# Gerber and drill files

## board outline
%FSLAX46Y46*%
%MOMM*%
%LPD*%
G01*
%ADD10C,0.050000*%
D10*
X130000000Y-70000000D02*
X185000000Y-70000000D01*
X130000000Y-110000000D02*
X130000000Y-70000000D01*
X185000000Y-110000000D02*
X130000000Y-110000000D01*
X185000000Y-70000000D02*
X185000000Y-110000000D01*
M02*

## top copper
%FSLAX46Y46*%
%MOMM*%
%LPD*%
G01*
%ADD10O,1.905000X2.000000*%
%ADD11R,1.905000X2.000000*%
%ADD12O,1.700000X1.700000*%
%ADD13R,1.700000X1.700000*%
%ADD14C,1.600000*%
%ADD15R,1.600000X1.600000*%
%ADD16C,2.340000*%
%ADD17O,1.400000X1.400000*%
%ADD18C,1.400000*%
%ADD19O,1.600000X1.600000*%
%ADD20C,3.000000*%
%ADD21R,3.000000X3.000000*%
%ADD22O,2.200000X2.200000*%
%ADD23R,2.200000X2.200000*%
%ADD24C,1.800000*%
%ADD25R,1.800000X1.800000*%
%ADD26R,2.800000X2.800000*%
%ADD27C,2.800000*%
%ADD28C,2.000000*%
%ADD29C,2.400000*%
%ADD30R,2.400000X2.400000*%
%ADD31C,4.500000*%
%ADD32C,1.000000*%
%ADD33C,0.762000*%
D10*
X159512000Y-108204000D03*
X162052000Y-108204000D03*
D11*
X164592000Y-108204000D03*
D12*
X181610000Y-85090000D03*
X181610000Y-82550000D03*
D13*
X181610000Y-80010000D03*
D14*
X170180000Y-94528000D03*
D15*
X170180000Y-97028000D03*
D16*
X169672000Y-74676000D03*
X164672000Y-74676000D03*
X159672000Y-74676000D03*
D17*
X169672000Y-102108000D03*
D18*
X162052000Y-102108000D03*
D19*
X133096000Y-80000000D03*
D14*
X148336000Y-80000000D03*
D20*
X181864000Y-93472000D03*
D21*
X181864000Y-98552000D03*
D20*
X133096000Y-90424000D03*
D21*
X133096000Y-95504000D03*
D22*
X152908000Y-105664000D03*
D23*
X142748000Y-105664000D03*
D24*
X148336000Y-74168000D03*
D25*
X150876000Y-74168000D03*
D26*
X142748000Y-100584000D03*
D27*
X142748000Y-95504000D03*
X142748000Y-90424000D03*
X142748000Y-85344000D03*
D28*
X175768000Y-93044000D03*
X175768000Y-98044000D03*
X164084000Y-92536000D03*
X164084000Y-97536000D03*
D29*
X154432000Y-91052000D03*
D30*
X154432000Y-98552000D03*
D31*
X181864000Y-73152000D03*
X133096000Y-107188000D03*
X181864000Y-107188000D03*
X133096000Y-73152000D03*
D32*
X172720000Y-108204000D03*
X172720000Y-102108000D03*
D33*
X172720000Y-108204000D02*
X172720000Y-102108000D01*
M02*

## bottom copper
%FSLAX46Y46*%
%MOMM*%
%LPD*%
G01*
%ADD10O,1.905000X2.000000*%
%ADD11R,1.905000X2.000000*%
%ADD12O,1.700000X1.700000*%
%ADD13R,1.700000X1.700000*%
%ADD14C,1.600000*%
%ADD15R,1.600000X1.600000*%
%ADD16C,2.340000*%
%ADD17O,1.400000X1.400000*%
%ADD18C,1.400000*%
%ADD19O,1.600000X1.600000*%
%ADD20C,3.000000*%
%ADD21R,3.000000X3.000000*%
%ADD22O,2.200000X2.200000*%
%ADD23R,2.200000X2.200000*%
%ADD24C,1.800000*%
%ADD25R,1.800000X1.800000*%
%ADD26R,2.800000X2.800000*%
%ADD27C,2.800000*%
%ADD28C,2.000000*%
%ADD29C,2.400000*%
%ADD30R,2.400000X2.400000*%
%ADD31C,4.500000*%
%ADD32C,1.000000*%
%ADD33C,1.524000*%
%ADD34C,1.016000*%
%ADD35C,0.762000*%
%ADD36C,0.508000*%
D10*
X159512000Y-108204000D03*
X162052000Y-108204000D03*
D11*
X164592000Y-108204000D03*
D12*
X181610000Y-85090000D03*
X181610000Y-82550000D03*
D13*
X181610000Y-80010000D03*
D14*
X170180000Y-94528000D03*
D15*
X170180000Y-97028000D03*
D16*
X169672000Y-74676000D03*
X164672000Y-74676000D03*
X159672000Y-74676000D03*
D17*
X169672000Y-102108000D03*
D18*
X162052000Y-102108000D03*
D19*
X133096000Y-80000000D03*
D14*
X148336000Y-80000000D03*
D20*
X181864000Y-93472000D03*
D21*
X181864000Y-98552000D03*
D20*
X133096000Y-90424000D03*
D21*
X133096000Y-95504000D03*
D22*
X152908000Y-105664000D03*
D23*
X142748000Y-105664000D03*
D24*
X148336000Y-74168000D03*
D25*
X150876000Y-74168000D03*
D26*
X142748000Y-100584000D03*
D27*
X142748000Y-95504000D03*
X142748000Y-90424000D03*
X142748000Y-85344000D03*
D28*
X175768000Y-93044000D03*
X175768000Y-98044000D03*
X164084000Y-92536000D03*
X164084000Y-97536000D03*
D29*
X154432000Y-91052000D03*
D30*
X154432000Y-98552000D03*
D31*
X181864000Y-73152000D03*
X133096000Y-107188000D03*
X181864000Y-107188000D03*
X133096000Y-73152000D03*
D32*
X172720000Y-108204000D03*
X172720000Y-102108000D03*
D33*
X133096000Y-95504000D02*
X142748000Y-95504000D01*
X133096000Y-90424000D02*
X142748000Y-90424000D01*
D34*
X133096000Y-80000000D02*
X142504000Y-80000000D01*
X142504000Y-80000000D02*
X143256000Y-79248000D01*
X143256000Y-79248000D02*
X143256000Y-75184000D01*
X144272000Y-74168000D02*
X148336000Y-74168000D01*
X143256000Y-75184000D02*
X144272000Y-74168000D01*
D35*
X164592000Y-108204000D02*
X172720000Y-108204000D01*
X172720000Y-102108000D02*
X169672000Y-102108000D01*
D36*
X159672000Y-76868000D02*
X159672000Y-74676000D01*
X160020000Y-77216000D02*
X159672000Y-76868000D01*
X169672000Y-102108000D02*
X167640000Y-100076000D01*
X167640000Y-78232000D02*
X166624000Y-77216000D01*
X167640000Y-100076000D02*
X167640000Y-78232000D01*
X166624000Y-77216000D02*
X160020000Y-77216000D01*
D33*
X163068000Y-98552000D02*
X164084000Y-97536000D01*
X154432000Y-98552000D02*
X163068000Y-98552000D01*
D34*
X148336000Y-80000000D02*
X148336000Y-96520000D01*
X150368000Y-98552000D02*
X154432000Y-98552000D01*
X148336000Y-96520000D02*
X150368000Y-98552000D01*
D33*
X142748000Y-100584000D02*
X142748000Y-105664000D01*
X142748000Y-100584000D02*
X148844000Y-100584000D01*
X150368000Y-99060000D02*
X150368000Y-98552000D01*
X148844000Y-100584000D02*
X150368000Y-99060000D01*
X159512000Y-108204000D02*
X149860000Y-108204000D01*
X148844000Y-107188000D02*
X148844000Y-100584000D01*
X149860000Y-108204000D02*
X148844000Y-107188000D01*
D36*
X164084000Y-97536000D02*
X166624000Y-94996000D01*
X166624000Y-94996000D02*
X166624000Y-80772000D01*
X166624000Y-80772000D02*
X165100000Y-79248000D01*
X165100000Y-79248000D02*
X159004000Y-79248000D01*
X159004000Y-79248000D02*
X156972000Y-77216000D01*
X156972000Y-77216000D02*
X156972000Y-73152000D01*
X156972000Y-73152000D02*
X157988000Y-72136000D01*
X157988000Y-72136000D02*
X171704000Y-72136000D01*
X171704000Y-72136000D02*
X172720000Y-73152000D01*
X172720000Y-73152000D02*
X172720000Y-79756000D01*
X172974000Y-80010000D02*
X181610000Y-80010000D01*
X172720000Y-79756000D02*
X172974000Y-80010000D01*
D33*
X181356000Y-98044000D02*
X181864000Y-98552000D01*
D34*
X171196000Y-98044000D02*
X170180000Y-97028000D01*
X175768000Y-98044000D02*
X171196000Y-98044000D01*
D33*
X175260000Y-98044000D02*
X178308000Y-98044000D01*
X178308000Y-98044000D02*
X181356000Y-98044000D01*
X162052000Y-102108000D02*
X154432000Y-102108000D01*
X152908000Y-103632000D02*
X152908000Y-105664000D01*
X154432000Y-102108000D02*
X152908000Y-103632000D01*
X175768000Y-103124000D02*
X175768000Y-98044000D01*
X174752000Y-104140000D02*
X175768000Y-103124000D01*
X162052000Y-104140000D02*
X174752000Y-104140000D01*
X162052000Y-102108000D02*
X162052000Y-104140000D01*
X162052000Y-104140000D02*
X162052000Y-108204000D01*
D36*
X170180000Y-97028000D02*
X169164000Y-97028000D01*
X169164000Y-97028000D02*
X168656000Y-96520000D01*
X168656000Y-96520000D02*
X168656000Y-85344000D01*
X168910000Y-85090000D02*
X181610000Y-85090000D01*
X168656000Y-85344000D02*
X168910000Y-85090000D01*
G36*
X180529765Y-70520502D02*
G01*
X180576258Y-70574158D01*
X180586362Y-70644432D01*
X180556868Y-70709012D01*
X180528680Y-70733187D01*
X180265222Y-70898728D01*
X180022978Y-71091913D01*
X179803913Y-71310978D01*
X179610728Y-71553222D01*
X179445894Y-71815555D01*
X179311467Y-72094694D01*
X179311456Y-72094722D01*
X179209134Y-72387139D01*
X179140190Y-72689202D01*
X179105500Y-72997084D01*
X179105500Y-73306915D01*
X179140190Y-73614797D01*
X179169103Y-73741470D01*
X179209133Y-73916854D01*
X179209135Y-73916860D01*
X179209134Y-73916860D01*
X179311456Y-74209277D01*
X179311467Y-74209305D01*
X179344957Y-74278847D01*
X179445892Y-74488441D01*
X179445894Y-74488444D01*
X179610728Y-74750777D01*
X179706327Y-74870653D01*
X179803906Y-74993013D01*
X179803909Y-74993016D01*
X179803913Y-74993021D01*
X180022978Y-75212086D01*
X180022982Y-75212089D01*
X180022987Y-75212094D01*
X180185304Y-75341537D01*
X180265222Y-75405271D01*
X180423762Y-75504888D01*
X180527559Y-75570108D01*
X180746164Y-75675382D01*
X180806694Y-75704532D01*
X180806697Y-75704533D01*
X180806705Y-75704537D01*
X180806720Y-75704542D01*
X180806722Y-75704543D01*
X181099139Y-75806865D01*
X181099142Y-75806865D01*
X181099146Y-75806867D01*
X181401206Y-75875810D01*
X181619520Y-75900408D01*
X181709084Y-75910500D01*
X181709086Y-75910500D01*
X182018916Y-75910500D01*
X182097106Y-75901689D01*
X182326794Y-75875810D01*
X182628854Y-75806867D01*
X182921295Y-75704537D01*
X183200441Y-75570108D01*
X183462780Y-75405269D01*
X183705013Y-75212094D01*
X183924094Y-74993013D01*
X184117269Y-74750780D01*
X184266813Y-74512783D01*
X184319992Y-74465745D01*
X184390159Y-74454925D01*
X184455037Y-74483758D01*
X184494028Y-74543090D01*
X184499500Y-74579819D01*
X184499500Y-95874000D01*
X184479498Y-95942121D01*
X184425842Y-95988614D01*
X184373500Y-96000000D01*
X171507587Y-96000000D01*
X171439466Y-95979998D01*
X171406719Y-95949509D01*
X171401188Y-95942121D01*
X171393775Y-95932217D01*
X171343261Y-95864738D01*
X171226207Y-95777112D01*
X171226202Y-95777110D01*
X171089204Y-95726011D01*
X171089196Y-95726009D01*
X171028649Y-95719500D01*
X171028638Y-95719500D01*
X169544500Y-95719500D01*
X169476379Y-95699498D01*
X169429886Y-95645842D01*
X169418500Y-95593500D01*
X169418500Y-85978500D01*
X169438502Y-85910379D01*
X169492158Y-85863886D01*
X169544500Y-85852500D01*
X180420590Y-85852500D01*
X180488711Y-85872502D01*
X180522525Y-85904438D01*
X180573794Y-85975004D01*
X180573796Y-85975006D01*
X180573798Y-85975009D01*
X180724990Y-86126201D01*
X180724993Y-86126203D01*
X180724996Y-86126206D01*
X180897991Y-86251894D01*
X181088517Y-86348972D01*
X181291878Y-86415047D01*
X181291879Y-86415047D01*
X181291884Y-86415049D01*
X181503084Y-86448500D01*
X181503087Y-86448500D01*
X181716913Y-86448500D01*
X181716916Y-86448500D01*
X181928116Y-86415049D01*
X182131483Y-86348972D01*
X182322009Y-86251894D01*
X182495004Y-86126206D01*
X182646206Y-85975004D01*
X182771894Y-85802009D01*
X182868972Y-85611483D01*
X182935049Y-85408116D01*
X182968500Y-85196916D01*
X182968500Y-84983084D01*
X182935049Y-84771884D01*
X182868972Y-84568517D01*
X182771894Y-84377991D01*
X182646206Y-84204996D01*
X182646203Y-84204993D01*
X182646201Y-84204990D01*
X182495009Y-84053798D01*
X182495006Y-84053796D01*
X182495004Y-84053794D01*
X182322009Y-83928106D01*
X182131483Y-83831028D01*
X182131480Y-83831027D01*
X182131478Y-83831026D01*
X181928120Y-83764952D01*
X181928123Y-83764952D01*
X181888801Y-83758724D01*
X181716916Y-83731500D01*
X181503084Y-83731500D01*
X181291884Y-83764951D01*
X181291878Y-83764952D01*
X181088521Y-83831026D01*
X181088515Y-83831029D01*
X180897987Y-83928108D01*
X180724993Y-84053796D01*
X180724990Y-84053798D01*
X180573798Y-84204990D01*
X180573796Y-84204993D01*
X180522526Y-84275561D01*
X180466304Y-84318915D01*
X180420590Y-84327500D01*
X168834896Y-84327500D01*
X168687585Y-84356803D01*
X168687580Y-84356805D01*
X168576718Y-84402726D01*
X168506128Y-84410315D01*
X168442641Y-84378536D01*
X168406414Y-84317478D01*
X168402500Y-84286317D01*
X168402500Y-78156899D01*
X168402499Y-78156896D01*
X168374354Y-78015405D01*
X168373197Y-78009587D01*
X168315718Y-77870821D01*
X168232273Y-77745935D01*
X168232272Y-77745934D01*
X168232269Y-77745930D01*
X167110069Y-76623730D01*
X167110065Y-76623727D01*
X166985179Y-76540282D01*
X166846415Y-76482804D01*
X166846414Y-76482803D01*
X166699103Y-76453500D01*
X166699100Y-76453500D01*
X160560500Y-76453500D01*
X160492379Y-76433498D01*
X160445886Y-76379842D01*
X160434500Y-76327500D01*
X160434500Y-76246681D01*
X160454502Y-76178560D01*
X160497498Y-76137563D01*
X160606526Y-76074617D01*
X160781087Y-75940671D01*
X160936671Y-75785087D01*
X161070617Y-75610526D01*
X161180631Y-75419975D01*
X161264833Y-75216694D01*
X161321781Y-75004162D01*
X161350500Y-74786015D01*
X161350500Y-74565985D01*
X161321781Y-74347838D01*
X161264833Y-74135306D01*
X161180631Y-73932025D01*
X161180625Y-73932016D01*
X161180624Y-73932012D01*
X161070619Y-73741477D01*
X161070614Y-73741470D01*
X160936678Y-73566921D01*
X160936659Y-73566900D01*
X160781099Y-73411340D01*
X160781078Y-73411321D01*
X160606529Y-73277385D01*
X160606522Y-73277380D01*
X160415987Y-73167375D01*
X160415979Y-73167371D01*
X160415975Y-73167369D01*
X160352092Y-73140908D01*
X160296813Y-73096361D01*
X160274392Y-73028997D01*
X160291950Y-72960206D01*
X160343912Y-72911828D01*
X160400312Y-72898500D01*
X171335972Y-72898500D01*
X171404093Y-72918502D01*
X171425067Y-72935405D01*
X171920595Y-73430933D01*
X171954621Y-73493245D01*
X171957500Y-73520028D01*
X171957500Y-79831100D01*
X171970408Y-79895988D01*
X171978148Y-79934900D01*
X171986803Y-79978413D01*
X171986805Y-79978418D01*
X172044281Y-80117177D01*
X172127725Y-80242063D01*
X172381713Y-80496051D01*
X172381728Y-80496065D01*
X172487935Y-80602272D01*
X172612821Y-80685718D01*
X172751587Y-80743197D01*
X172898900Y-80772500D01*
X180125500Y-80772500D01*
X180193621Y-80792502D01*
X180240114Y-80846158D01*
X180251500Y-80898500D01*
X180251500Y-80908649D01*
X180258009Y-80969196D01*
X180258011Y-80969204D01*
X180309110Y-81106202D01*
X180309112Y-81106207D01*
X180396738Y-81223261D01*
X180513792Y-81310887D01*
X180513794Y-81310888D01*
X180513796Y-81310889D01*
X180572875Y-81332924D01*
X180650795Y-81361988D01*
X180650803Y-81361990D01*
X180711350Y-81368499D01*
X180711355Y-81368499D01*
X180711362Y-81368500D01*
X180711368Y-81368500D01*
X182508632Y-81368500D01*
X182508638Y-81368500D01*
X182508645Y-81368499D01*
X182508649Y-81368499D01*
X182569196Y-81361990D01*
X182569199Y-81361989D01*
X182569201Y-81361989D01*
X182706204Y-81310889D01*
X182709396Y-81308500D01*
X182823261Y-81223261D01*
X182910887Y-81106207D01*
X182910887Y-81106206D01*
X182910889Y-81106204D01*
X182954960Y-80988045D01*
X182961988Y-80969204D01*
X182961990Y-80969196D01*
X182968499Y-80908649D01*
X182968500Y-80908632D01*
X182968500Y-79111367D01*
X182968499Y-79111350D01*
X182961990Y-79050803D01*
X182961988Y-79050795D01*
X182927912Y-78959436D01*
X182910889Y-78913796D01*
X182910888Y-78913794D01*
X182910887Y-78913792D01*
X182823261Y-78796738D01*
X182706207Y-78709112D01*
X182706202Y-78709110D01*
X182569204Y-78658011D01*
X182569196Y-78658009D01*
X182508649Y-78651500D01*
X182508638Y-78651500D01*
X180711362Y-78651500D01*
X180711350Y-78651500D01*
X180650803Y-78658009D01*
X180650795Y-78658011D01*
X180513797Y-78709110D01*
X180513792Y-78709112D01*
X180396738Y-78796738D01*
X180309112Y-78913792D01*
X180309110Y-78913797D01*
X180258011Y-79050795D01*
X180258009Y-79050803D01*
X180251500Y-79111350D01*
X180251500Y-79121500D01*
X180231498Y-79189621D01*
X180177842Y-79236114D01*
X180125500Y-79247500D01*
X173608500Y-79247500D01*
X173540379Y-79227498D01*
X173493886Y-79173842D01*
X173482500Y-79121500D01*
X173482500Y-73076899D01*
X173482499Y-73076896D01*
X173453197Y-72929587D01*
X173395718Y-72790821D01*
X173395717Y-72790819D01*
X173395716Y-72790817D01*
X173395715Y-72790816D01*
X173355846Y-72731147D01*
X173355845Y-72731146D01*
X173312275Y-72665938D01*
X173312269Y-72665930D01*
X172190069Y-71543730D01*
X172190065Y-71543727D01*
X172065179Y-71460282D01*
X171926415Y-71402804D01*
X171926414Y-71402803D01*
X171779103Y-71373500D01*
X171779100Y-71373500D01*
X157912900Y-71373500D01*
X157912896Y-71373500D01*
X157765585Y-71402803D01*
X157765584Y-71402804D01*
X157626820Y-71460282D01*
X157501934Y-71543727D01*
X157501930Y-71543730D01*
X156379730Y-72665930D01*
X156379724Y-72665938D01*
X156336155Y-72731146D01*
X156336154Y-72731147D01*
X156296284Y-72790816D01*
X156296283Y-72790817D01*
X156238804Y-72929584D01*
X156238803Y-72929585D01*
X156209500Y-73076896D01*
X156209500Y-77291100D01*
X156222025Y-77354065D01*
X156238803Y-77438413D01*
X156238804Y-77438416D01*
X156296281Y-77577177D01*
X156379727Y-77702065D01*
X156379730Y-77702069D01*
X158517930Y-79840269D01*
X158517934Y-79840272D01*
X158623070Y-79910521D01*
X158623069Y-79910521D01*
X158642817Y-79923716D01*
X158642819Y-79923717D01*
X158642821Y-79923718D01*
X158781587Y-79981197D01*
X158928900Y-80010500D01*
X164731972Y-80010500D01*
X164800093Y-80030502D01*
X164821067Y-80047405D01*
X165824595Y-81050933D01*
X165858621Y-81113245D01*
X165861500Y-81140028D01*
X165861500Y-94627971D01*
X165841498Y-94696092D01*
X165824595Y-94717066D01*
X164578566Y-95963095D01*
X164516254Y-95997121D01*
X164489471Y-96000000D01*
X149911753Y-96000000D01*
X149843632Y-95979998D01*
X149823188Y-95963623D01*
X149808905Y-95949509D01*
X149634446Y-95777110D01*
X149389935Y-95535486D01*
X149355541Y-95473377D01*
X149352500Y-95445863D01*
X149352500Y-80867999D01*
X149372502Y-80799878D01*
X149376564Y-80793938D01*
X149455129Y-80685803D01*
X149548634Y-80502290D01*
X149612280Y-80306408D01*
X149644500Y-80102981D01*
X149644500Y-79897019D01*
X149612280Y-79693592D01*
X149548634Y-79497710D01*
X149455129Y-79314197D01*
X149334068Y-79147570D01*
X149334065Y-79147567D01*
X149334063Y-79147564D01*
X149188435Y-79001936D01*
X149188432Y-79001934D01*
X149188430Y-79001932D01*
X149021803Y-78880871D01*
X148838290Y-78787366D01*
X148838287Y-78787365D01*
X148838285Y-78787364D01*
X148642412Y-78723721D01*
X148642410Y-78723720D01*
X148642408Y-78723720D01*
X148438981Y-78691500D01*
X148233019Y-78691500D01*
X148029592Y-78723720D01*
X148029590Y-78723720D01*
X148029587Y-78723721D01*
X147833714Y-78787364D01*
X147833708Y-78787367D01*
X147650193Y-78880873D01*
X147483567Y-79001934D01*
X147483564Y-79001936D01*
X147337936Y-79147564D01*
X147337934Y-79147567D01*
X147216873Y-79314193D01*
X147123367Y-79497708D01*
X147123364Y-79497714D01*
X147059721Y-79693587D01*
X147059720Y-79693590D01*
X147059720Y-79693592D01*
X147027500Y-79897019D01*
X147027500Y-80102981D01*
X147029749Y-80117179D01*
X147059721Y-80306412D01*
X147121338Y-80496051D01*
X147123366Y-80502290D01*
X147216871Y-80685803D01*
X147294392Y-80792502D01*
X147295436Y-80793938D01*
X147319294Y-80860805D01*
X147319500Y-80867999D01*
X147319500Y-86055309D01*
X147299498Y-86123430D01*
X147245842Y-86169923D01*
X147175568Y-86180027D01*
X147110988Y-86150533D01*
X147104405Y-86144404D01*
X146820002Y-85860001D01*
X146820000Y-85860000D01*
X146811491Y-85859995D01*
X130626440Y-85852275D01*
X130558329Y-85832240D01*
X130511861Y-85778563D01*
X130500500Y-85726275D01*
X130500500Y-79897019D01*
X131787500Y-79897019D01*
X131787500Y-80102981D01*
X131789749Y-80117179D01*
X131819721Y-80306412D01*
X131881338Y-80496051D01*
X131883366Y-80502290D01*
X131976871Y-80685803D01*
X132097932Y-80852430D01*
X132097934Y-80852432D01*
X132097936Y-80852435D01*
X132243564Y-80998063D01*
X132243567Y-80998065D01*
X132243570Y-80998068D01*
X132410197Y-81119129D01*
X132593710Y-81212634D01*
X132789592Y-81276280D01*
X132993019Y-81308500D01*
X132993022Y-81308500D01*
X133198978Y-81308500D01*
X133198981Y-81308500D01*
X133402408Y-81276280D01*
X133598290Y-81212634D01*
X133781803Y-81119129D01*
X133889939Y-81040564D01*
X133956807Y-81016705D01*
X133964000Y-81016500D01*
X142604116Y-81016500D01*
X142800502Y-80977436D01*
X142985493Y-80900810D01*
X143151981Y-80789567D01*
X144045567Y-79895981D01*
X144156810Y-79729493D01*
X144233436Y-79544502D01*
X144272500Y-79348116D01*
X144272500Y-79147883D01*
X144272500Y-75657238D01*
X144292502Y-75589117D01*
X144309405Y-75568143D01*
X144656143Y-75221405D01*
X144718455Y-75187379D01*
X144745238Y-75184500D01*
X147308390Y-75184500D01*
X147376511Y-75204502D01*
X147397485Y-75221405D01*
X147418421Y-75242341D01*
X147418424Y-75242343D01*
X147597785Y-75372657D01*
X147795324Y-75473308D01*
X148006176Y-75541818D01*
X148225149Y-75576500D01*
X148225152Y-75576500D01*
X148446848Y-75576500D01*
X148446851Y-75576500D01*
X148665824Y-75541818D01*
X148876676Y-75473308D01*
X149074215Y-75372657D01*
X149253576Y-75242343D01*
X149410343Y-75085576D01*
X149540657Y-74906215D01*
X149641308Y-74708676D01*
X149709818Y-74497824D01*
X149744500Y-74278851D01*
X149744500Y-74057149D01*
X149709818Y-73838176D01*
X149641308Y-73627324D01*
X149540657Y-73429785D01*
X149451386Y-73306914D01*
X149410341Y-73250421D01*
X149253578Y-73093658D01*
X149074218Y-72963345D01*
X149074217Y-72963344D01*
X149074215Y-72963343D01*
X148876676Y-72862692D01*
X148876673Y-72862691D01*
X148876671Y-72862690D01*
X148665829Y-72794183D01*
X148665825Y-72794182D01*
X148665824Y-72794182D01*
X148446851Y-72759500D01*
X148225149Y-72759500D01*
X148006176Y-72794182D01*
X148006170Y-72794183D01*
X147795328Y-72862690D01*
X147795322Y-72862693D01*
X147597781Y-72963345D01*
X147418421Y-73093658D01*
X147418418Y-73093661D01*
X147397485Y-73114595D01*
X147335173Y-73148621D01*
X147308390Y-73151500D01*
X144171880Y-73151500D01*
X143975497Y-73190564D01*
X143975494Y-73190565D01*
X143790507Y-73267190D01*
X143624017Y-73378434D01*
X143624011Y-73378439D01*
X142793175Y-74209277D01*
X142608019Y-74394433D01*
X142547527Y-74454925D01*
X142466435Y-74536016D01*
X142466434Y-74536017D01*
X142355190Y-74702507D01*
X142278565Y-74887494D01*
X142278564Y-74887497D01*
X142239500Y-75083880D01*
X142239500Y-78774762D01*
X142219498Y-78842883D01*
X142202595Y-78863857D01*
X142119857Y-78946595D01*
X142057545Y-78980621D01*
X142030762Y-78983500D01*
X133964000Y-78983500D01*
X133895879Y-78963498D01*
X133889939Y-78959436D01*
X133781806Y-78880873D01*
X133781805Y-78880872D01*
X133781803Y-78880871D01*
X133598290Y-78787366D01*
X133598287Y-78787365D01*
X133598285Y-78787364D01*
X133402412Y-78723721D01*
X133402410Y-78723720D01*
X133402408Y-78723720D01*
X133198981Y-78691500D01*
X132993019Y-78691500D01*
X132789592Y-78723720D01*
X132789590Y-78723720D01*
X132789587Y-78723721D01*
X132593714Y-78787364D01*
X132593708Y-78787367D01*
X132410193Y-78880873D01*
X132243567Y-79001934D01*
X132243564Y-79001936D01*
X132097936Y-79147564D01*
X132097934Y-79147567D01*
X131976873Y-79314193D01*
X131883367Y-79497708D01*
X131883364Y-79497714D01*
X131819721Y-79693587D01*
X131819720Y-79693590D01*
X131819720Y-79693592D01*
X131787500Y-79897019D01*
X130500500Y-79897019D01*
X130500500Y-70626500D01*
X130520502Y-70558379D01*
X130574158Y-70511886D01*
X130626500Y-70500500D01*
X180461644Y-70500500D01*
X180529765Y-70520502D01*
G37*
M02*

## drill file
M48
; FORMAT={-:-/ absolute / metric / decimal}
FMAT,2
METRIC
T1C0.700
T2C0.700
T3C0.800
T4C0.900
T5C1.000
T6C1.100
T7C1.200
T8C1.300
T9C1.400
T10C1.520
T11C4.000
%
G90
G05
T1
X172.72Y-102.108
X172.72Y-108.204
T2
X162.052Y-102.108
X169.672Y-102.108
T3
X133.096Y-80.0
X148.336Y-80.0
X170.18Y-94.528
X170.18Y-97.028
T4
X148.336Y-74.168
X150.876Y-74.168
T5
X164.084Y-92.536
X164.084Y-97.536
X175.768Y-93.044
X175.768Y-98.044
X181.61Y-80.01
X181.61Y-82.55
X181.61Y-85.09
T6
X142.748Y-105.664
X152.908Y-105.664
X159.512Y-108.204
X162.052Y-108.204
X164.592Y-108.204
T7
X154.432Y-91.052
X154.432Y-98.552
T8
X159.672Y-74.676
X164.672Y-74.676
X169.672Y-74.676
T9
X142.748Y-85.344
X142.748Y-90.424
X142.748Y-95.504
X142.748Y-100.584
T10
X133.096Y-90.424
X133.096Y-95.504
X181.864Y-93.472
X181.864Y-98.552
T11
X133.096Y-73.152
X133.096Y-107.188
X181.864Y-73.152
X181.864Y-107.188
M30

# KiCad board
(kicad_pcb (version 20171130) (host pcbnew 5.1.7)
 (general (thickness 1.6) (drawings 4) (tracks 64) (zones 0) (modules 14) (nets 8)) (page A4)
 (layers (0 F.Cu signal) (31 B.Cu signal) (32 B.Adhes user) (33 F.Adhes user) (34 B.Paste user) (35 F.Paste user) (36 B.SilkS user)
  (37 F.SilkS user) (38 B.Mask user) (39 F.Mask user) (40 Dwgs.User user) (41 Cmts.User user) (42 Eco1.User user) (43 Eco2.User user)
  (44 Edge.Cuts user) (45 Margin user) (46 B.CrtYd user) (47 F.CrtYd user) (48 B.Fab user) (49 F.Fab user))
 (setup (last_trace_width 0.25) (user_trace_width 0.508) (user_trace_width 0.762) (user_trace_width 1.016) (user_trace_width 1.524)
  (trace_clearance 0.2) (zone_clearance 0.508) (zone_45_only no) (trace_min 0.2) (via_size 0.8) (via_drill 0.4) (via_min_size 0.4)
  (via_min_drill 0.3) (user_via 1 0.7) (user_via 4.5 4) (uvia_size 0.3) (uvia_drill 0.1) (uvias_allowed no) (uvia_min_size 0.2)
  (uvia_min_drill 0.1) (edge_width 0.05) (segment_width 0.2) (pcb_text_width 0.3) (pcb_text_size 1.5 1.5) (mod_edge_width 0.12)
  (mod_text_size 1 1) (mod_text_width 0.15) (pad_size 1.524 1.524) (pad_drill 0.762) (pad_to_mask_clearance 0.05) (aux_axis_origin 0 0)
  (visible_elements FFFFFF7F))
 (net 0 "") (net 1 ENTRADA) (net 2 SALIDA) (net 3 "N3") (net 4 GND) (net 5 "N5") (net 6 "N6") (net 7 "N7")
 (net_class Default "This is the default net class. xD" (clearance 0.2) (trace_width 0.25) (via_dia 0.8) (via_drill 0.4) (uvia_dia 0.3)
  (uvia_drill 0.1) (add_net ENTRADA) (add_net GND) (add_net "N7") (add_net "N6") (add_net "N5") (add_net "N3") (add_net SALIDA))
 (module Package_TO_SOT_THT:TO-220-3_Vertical (layer F.Cu) (at 164.592 108.204 180)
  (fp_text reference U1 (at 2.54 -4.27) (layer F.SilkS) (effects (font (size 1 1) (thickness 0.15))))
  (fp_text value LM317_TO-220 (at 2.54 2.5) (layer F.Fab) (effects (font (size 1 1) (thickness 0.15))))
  (pad 3 thru_hole oval (at 5.08 0 180) (size 1.905 2) (drill 1.1) (layers *.Cu *.Mask) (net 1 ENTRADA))
  (pad 2 thru_hole oval (at 2.54 0 180) (size 1.905 2) (drill 1.1) (layers *.Cu *.Mask) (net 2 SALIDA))
  (pad 1 thru_hole rect (at 0 0 180) (size 1.905 2) (drill 1.1) (layers *.Cu *.Mask) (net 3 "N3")))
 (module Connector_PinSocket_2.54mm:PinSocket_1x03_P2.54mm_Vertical (layer F.Cu) (at 181.61 80.01)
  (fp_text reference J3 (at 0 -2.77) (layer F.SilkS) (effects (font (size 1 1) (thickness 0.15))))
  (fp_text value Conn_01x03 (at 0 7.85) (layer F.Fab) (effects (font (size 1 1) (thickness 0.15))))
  (pad 3 thru_hole oval (at 0 5.08) (size 1.7 1.7) (drill 1) (layers *.Cu *.Mask) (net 2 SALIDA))
  (pad 2 thru_hole oval (at 0 2.54) (size 1.7 1.7) (drill 1) (layers *.Cu *.Mask) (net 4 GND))
  (pad 1 thru_hole rect (at 0 0) (size 1.7 1.7) (drill 1) (layers *.Cu *.Mask) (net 1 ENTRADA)))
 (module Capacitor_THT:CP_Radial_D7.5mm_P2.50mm (layer F.Cu) (at 170.18 97.028 90)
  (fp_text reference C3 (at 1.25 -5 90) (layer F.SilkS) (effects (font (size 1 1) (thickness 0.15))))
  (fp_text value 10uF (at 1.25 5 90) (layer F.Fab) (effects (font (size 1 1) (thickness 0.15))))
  (pad 2 thru_hole circle (at 2.5 0 90) (size 1.6 1.6) (drill 0.8) (layers *.Cu *.Mask) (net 4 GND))
  (pad 1 thru_hole rect (at 0 0 90) (size 1.6 1.6) (drill 0.8) (layers *.Cu *.Mask) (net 2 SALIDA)))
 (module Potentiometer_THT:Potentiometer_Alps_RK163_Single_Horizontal (layer F.Cu) (at 169.672 74.676 90)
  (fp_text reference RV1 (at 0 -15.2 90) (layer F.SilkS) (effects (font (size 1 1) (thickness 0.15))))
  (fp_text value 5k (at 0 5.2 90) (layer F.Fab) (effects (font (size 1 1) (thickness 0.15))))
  (pad 1 thru_hole circle (at 0 0 90) (size 2.34 2.34) (drill 1.3) (layers *.Cu *.Mask) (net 4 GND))
  (pad 2 thru_hole circle (at 0 -5 90) (size 2.34 2.34) (drill 1.3) (layers *.Cu *.Mask) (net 4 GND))
  (pad 3 thru_hole circle (at 0 -10 90) (size 2.34 2.34) (drill 1.3) (layers *.Cu *.Mask) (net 3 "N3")))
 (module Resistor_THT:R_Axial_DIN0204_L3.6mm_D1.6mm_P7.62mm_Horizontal (layer F.Cu) (at 162.052 102.108)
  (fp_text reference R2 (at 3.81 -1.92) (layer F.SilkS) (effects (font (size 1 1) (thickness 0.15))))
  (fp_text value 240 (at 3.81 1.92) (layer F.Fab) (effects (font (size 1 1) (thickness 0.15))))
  (pad 2 thru_hole oval (at 7.62 0) (size 1.4 1.4) (drill 0.7) (layers *.Cu *.Mask) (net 3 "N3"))
  (pad 1 thru_hole circle (at 0 0) (size 1.4 1.4) (drill 0.7) (layers *.Cu *.Mask) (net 2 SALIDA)))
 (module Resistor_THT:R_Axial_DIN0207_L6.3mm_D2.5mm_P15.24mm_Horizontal (layer F.Cu) (at 148.336 80 180)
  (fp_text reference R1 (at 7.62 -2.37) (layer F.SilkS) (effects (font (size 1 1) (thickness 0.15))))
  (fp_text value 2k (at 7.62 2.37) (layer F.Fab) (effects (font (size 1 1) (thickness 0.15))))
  (pad 2 thru_hole oval (at 15.24 0 180) (size 1.6 1.6) (drill 0.8) (layers *.Cu *.Mask) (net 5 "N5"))
  (pad 1 thru_hole circle (at 0 0 180) (size 1.6 1.6) (drill 0.8) (layers *.Cu *.Mask) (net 1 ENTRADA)))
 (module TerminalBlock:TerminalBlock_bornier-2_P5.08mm (layer F.Cu) (at 181.864 98.552 90)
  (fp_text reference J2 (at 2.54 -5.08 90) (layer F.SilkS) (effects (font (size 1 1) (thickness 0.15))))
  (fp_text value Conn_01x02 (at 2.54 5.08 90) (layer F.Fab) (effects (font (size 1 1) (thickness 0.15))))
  (pad 2 thru_hole circle (at 5.08 0 90) (size 3 3) (drill 1.52) (layers *.Cu *.Mask) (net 4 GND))
  (pad 1 thru_hole rect (at 0 0 90) (size 3 3) (drill 1.52) (layers *.Cu *.Mask) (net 2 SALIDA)))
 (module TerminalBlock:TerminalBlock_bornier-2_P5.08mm (layer F.Cu) (at 133.096 95.504 90)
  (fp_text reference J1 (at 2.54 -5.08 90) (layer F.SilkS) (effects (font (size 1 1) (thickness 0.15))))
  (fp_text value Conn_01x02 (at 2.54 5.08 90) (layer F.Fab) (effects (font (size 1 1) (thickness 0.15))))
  (pad 2 thru_hole circle (at 5.08 0 90) (size 3 3) (drill 1.52) (layers *.Cu *.Mask) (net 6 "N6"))
  (pad 1 thru_hole rect (at 0 0 90) (size 3 3) (drill 1.52) (layers *.Cu *.Mask) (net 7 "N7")))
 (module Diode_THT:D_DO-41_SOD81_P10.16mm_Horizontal (layer F.Cu) (at 142.748 105.664)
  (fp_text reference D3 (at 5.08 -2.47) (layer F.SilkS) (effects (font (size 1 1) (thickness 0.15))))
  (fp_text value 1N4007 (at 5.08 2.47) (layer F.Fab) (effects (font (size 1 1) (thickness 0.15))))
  (pad 2 thru_hole oval (at 10.16 0) (size 2.2 2.2) (drill 1.1) (layers *.Cu *.Mask) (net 2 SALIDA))
  (pad 1 thru_hole rect (at 0 0) (size 2.2 2.2) (drill 1.1) (layers *.Cu *.Mask) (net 1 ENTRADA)))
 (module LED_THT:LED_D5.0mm (layer F.Cu) (at 150.876 74.168 180)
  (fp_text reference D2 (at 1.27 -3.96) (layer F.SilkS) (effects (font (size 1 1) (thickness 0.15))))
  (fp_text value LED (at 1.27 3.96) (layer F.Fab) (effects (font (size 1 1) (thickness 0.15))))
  (pad 2 thru_hole circle (at 2.54 0 180) (size 1.8 1.8) (drill 0.9) (layers *.Cu *.Mask) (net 5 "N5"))
  (pad 1 thru_hole rect (at 0 0 180) (size 1.8 1.8) (drill 0.9) (layers *.Cu *.Mask) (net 4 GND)))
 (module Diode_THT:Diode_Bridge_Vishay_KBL (layer F.Cu) (at 142.748 100.584 90)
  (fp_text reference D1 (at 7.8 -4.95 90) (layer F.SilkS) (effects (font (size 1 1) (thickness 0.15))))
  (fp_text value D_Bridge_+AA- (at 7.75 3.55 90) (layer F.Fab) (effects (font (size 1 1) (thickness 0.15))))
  (pad 1 thru_hole rect (at 0 0 90) (size 2.8 2.8) (drill 1.4) (layers *.Cu *.Mask) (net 1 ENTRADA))
  (pad 2 thru_hole circle (at 5.08 0 90) (size 2.8 2.8) (drill 1.4) (layers *.Cu *.Mask) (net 7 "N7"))
  (pad 3 thru_hole circle (at 10.16 0 90) (size 2.8 2.8) (drill 1.4) (layers *.Cu *.Mask) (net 6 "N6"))
  (pad 4 thru_hole circle (at 15.24 0 90) (size 2.8 2.8) (drill 1.4) (layers *.Cu *.Mask) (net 4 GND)))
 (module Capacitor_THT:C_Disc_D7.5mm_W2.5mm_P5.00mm (layer F.Cu) (at 175.768 98.044 90)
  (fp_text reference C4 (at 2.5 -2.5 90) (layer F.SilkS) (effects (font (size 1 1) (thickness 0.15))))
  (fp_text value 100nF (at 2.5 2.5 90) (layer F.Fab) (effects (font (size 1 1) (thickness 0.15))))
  (pad 2 thru_hole circle (at 5 0 90) (size 2 2) (drill 1) (layers *.Cu *.Mask) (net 4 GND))
  (pad 1 thru_hole circle (at 0 0 90) (size 2 2) (drill 1) (layers *.Cu *.Mask) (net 2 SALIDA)))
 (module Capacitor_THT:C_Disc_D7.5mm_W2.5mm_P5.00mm (layer F.Cu) (at 164.084 97.536 90)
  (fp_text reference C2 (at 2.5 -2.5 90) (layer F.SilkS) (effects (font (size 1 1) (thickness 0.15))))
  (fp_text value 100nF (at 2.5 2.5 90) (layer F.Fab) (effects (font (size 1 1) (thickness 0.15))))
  (pad 2 thru_hole circle (at 5 0 90) (size 2 2) (drill 1) (layers *.Cu *.Mask) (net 4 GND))
  (pad 1 thru_hole circle (at 0 0 90) (size 2 2) (drill 1) (layers *.Cu *.Mask) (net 1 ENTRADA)))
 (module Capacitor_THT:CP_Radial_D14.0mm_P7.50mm (layer F.Cu) (at 154.432 98.552 90)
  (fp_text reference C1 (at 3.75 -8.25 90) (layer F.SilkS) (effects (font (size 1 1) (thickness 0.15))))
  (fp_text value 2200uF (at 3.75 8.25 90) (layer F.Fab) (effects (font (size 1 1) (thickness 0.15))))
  (pad 2 thru_hole circle (at 7.5 0 90) (size 2.4 2.4) (drill 1.2) (layers *.Cu *.Mask) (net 4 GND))
  (pad 1 thru_hole rect (at 0 0 90) (size 2.4 2.4) (drill 1.2) (layers *.Cu *.Mask) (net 1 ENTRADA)))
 (gr_line (start 130 70) (end 185 70) (layer Edge.Cuts) (width 0.05))
 (gr_line (start 130 110) (end 130 70) (layer Edge.Cuts) (width 0.05))
 (gr_line (start 185 110) (end 130 110) (layer Edge.Cuts) (width 0.05))
 (gr_line (start 185 70) (end 185 110) (layer Edge.Cuts) (width 0.05))
 (via (at 181.864 73.152) (size 4.5) (drill 4) (layers F.Cu B.Cu) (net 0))
 (via (at 133.096 107.188) (size 4.5) (drill 4) (layers F.Cu B.Cu) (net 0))
 (via (at 181.864 107.188) (size 4.5) (drill 4) (layers F.Cu B.Cu) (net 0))
 (via (at 133.096 73.152) (size 4.5) (drill 4) (layers F.Cu B.Cu) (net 4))
 (segment (start 133.096 95.504) (end 142.748 95.504) (width 1.524) (layer B.Cu) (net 7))
 (segment (start 133.096 90.424) (end 142.748 90.424) (width 1.524) (layer B.Cu) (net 6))
 (segment (start 133.096 80) (end 142.504 80) (width 1.016) (layer B.Cu) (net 5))
 (segment (start 142.504 80) (end 143.256 79.248) (width 1.016) (layer B.Cu) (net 5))
 (segment (start 143.256 79.248) (end 143.256 75.184) (width 1.016) (layer B.Cu) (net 5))
 (segment (start 144.272 74.168) (end 148.336 74.168) (width 1.016) (layer B.Cu) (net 5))
 (segment (start 143.256 75.184) (end 144.272 74.168) (width 1.016) (layer B.Cu) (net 5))
 (segment (start 164.592 108.204) (end 172.72 108.204) (width 0.762) (layer B.Cu) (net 3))
 (via (at 172.72 108.204) (size 1) (drill 0.7) (layers F.Cu B.Cu) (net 3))
 (segment (start 172.72 108.204) (end 172.72 102.108) (width 0.762) (layer F.Cu) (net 3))
 (via (at 172.72 102.108) (size 1) (drill 0.7) (layers F.Cu B.Cu) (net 3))
 (segment (start 172.72 102.108) (end 169.672 102.108) (width 0.762) (layer B.Cu) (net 3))
 (segment (start 159.672 76.868) (end 159.672 74.676) (width 0.508) (layer B.Cu) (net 3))
 (segment (start 160.02 77.216) (end 159.672 76.868) (width 0.508) (layer B.Cu) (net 3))
 (segment (start 169.672 102.108) (end 167.64 100.076) (width 0.508) (layer B.Cu) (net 3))
 (segment (start 167.64 78.232) (end 166.624 77.216) (width 0.508) (layer B.Cu) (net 3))
 (segment (start 167.64 100.076) (end 167.64 78.232) (width 0.508) (layer B.Cu) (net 3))
 (segment (start 166.624 77.216) (end 160.02 77.216) (width 0.508) (layer B.Cu) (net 3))
 (segment (start 163.068 98.552) (end 164.084 97.536) (width 1.524) (layer B.Cu) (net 1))
 (segment (start 154.432 98.552) (end 163.068 98.552) (width 1.524) (layer B.Cu) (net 1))
 (segment (start 148.336 80) (end 148.336 96.52) (width 1.016) (layer B.Cu) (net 1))
 (segment (start 150.368 98.552) (end 154.432 98.552) (width 1.016) (layer B.Cu) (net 1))
 (segment (start 148.336 96.52) (end 150.368 98.552) (width 1.016) (layer B.Cu) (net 1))
 (segment (start 142.748 100.584) (end 142.748 105.664) (width 1.524) (layer B.Cu) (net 1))
 (segment (start 142.748 100.584) (end 148.844 100.584) (width 1.524) (layer B.Cu) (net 1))
 (segment (start 150.368 99.06) (end 150.368 98.552) (width 1.524) (layer B.Cu) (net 1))
 (segment (start 148.844 100.584) (end 150.368 99.06) (width 1.524) (layer B.Cu) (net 1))
 (segment (start 159.512 108.204) (end 149.86 108.204) (width 1.524) (layer B.Cu) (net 1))
 (segment (start 148.844 107.188) (end 148.844 100.584) (width 1.524) (layer B.Cu) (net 1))
 (segment (start 149.86 108.204) (end 148.844 107.188) (width 1.524) (layer B.Cu) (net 1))
 (segment (start 164.084 97.536) (end 166.624 94.996) (width 0.508) (layer B.Cu) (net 1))
 (segment (start 166.624 94.996) (end 166.624 80.772) (width 0.508) (layer B.Cu) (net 1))
 (segment (start 166.624 80.772) (end 165.1 79.248) (width 0.508) (layer B.Cu) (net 1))
 (segment (start 165.1 79.248) (end 159.004 79.248) (width 0.508) (layer B.Cu) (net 1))
 (segment (start 159.004 79.248) (end 156.972 77.216) (width 0.508) (layer B.Cu) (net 1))
 (segment (start 156.972 77.216) (end 156.972 73.152) (width 0.508) (layer B.Cu) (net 1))
 (segment (start 156.972 73.152) (end 157.988 72.136) (width 0.508) (layer B.Cu) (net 1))
 (segment (start 157.988 72.136) (end 171.704 72.136) (width 0.508) (layer B.Cu) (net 1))
 (segment (start 171.704 72.136) (end 172.72 73.152) (width 0.508) (layer B.Cu) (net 1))
 (segment (start 172.72 73.152) (end 172.72 79.756) (width 0.508) (layer B.Cu) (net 1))
 (segment (start 172.974 80.01) (end 181.61 80.01) (width 0.508) (layer B.Cu) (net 1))
 (segment (start 172.72 79.756) (end 172.974 80.01) (width 0.508) (layer B.Cu) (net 1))
 (segment (start 181.356 98.044) (end 181.864 98.552) (width 1.524) (layer B.Cu) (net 2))
 (segment (start 171.196 98.044) (end 170.18 97.028) (width 1.016) (layer B.Cu) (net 2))
 (segment (start 175.768 98.044) (end 171.196 98.044) (width 1.016) (layer B.Cu) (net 2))
 (segment (start 175.26 98.044) (end 178.308 98.044) (width 1.524) (layer B.Cu) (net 2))
 (segment (start 178.308 98.044) (end 181.356 98.044) (width 1.524) (layer B.Cu) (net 2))
 (segment (start 162.052 102.108) (end 154.432 102.108) (width 1.524) (layer B.Cu) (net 2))
 (segment (start 152.908 103.632) (end 152.908 105.664) (width 1.524) (layer B.Cu) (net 2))
 (segment (start 154.432 102.108) (end 152.908 103.632) (width 1.524) (layer B.Cu) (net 2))
 (segment (start 175.768 103.124) (end 175.768 98.044) (width 1.524) (layer B.Cu) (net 2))
 (segment (start 174.752 104.14) (end 175.768 103.124) (width 1.524) (layer B.Cu) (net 2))
 (segment (start 162.052 104.14) (end 174.752 104.14) (width 1.524) (layer B.Cu) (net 2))
 (segment (start 162.052 102.108) (end 162.052 104.14) (width 1.524) (layer B.Cu) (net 2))
 (segment (start 162.052 104.14) (end 162.052 108.204) (width 1.524) (layer B.Cu) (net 2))
 (segment (start 170.18 97.028) (end 169.164 97.028) (width 0.508) (layer B.Cu) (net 2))
 (segment (start 169.164 97.028) (end 168.656 96.52) (width 0.508) (layer B.Cu) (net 2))
 (segment (start 168.656 96.52) (end 168.656 85.344) (width 0.508) (layer B.Cu) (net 2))
 (segment (start 168.91 85.09) (end 181.61 85.09) (width 0.508) (layer B.Cu) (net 2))
 (segment (start 168.656 85.344) (end 168.91 85.09) (width 0.508) (layer B.Cu) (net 2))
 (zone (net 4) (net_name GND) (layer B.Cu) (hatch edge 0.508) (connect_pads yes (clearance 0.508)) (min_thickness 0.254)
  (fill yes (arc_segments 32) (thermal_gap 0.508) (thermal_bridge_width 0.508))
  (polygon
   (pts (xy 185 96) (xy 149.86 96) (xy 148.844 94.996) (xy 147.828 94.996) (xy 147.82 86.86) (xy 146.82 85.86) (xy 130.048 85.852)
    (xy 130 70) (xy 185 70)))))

